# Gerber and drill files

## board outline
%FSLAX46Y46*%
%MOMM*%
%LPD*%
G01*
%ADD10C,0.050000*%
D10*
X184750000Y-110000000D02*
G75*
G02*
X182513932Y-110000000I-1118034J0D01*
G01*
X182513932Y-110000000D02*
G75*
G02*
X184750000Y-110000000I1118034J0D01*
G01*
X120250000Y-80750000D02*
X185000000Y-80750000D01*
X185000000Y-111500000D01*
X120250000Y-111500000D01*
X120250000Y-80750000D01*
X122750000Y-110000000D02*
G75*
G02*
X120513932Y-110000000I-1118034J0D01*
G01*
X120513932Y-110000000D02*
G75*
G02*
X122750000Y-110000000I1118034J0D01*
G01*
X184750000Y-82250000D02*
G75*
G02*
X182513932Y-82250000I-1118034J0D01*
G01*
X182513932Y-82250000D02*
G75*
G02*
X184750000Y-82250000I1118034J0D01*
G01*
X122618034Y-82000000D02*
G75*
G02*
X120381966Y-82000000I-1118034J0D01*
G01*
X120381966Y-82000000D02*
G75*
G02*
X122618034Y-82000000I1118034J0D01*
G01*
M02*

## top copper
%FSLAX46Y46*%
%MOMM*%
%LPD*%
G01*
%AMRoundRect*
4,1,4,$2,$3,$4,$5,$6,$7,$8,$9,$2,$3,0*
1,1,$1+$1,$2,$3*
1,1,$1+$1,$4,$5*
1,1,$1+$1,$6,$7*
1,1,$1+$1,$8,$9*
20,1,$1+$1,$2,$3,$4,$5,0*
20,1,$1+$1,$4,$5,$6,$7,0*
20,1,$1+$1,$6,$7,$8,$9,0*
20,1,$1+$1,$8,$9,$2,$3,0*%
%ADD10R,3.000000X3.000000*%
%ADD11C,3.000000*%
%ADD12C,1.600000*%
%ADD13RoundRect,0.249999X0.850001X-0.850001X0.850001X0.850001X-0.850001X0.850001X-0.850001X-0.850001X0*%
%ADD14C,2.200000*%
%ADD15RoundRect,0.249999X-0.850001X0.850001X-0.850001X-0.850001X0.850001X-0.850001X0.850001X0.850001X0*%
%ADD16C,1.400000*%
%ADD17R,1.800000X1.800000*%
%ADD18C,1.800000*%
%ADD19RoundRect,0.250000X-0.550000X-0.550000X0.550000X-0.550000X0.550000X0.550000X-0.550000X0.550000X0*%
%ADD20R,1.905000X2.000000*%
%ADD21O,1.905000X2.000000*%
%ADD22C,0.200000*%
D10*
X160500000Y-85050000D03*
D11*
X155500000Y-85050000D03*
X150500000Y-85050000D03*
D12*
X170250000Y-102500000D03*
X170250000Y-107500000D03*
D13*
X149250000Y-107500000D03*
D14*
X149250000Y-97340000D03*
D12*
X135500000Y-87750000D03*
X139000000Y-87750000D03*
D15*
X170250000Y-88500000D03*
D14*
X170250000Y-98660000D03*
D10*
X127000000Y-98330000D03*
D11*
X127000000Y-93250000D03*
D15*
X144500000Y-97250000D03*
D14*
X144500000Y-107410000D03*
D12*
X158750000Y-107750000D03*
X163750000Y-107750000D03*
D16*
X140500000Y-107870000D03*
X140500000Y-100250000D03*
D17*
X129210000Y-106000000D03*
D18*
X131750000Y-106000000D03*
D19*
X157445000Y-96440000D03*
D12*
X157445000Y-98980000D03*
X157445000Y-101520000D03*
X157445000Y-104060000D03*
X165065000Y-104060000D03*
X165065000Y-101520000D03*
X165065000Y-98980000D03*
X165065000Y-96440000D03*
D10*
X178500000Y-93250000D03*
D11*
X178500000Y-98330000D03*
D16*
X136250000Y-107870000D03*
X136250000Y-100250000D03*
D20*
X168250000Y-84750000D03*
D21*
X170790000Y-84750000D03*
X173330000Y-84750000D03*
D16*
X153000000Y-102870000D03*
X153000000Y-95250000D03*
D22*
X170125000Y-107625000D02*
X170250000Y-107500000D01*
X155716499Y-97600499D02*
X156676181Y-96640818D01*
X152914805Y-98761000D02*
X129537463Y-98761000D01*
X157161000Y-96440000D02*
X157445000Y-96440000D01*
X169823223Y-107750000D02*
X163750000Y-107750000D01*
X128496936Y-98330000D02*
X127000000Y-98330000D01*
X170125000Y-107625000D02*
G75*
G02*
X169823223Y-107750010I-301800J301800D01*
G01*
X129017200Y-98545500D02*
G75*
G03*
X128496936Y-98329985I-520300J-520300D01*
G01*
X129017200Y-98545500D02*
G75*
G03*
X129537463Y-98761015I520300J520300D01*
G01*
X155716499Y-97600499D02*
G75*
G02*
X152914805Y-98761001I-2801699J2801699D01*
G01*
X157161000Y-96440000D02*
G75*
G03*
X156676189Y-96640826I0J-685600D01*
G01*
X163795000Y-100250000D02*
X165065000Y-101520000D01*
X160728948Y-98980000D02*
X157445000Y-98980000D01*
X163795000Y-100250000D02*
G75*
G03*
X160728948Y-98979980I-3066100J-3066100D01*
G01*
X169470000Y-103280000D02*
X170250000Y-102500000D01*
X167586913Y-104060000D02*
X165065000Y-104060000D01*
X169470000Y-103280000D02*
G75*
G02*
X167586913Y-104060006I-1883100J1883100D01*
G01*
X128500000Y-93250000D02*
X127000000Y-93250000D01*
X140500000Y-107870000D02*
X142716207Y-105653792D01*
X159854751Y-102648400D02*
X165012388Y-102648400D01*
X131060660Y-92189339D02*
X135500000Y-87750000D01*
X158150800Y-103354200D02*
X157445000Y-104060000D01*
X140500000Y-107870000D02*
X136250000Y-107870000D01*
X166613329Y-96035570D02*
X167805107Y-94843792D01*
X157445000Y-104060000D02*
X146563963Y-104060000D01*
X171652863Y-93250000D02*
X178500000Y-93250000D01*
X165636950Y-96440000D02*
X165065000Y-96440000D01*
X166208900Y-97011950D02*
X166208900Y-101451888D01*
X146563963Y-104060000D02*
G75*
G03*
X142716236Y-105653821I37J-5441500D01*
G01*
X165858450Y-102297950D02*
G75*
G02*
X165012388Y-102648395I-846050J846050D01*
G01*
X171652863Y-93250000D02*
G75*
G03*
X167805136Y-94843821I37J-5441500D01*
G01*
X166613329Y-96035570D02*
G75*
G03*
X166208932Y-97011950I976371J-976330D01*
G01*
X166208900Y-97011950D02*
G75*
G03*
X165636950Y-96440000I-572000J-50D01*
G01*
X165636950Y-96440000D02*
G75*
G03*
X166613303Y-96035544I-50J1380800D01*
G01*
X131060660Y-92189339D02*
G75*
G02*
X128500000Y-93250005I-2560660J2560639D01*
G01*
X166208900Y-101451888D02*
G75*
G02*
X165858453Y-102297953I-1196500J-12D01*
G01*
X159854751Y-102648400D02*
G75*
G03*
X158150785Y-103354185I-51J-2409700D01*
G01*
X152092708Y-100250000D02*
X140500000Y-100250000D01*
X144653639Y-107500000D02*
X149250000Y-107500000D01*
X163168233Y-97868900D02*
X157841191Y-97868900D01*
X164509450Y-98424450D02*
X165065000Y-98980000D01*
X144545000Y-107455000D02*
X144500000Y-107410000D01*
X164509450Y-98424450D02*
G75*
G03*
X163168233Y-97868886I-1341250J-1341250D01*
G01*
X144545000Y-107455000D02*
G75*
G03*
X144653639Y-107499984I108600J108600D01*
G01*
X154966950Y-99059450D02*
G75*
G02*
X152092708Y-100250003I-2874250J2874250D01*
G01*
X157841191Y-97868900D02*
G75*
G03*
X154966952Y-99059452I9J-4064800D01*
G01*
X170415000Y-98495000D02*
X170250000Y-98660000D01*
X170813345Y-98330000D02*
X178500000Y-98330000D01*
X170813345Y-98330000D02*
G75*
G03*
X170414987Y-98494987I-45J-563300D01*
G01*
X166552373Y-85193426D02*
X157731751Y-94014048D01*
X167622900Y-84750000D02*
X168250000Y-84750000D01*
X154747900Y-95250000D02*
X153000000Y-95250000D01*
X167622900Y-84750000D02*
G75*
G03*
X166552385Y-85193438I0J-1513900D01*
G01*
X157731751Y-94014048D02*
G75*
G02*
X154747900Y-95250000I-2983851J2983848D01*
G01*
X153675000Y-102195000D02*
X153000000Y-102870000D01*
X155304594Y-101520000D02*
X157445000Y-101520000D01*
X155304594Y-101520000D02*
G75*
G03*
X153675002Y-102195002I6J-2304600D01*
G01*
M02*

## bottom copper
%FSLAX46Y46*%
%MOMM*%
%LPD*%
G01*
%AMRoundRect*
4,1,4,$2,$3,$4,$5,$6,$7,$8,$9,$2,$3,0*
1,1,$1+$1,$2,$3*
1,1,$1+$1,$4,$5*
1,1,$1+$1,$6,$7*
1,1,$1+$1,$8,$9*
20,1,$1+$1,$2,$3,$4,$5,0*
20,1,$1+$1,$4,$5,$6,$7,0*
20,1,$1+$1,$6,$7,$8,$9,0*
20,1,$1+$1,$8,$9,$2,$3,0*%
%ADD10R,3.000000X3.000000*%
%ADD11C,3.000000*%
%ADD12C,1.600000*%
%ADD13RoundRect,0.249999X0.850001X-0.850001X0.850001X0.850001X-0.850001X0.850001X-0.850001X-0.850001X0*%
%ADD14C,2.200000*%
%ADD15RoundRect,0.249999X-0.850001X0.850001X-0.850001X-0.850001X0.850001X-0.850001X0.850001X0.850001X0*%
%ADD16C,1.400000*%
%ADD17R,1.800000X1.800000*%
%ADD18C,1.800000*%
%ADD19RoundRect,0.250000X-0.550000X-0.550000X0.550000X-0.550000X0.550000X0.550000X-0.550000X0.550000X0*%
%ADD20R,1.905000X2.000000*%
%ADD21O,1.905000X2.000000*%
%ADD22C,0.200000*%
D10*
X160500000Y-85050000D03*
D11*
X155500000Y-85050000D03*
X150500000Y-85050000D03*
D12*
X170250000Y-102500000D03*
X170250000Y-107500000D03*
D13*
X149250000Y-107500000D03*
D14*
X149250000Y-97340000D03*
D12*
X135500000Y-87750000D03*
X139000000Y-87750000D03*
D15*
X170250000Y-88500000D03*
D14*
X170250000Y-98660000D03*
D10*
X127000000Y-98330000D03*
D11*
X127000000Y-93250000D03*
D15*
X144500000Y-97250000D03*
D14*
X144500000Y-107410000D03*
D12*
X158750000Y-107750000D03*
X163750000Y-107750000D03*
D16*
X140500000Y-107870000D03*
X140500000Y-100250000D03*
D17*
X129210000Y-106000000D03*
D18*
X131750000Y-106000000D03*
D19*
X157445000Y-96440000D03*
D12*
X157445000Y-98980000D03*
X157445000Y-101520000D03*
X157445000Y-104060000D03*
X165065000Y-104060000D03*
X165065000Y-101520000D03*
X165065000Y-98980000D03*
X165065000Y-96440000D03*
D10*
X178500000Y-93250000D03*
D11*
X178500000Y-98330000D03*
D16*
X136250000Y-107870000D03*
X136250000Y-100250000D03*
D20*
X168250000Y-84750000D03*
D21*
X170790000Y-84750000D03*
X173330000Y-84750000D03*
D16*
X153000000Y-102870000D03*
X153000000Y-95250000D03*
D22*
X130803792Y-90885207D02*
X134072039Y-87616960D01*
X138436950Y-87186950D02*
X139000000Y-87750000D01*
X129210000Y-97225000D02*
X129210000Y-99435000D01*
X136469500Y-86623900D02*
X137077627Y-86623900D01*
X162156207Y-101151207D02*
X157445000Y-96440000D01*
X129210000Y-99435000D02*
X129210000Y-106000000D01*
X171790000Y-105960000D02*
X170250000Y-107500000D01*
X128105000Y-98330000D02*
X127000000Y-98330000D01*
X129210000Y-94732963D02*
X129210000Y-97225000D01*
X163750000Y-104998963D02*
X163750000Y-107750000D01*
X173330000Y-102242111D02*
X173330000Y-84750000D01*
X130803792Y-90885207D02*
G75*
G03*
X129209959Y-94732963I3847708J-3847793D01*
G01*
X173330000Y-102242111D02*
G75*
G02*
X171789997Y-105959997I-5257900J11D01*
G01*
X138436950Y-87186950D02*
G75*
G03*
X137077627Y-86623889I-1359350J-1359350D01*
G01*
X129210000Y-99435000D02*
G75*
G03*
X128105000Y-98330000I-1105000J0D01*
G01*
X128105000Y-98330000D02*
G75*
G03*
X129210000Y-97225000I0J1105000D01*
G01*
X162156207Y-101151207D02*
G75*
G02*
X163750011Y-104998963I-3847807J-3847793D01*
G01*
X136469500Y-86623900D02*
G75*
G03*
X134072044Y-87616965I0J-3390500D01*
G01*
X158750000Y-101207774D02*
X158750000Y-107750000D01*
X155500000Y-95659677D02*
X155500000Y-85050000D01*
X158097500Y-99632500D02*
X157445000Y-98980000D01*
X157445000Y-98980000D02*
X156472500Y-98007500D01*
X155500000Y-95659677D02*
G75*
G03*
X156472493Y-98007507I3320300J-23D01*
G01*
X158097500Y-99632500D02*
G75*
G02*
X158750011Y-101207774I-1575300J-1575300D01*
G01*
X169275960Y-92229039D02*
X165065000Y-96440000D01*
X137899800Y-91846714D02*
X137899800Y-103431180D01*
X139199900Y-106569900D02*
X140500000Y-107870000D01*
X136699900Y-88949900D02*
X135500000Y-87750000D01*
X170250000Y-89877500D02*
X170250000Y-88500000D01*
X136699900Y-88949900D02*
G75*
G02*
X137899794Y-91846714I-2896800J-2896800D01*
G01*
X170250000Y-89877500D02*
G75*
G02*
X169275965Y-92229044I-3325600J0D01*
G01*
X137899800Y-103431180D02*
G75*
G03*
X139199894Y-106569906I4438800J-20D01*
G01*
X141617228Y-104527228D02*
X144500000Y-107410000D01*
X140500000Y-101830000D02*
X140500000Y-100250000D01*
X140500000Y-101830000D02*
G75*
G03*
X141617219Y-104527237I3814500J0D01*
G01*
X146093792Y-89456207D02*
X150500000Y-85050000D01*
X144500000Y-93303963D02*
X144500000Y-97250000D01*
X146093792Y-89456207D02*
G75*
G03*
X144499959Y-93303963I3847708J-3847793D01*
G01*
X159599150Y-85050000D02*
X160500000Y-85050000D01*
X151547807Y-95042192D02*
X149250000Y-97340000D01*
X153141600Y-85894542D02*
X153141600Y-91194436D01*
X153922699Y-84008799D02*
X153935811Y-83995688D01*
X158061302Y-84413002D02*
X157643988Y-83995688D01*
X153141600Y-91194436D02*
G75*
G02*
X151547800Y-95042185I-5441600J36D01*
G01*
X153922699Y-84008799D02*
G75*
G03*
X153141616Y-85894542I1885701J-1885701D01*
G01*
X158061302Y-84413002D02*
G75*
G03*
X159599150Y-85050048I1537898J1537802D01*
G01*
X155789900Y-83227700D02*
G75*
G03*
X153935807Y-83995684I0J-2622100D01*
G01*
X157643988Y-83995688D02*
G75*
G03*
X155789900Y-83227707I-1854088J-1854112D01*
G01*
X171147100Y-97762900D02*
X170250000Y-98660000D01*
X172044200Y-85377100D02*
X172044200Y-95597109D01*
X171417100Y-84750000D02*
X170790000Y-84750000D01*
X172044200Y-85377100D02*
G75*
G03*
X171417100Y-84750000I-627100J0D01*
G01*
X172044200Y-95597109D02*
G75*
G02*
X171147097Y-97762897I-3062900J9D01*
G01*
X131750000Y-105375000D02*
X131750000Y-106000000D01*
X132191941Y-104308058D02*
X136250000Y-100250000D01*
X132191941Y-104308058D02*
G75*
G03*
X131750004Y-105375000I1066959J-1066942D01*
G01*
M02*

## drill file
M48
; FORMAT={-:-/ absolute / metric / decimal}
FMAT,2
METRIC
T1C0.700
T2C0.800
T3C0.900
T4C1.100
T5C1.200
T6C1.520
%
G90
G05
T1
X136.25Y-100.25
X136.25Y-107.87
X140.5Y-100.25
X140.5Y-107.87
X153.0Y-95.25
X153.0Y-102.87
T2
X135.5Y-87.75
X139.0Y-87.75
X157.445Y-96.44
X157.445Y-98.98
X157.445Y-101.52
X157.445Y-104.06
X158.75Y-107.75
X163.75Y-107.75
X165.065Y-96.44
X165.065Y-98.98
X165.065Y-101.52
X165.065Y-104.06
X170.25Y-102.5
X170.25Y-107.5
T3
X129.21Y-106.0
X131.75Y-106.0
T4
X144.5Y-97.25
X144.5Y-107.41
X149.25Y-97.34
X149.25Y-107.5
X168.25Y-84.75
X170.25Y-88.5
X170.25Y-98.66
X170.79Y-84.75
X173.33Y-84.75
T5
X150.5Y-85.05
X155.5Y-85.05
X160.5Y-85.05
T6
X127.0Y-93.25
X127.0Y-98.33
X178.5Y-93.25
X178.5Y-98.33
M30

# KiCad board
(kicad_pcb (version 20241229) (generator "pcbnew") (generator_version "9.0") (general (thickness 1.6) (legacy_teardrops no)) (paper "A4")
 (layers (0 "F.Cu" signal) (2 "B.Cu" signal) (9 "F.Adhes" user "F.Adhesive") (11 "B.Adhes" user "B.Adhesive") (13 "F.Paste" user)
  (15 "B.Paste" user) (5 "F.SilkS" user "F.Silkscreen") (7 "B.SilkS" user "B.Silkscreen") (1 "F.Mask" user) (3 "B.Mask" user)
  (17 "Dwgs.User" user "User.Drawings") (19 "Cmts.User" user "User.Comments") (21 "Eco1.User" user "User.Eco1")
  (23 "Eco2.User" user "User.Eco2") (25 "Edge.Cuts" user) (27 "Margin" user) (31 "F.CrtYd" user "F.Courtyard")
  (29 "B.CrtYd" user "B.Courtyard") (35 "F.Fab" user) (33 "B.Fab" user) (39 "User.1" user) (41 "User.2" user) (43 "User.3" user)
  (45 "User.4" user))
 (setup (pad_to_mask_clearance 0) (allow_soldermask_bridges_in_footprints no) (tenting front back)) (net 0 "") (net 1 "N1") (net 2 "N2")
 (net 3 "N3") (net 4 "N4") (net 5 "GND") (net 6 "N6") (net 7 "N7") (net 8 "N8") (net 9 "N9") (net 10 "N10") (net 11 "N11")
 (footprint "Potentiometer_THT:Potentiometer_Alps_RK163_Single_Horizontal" (layer "F.Cu") (at 160.5 85.05 -90)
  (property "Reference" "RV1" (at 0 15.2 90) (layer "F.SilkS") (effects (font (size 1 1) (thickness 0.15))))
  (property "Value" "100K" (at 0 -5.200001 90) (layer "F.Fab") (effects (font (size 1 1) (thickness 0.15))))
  (pad "1" thru_hole rect (at 0 0 90) (size 3 3) (drill 1.2) (layers "*.Cu" "*.Mask") (remove_unused_layers no) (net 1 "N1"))
  (pad "2" thru_hole circle (at 0 5 90) (size 3 3) (drill 1.2) (layers "*.Cu" "*.Mask") (remove_unused_layers no) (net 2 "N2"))
  (pad "3" thru_hole circle (at 0 10 90) (size 3 3) (drill 1.2) (layers "*.Cu" "*.Mask") (remove_unused_layers no) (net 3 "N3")))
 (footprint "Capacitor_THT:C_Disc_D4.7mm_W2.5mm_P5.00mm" (layer "F.Cu") (at 170.25 102.5 -90)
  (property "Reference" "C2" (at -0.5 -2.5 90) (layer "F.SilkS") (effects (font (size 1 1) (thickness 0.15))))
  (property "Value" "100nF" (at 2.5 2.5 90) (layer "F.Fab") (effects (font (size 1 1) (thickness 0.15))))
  (pad "1" thru_hole circle (at 0 0 270) (size 1.6 1.6) (drill 0.8) (layers "*.Cu" "*.Mask") (remove_unused_layers no) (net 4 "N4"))
  (pad "2" thru_hole circle (at 5 0 270) (size 1.6 1.6) (drill 0.8) (layers "*.Cu" "*.Mask") (remove_unused_layers no) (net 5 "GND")))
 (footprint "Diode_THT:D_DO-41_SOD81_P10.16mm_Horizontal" (layer "F.Cu") (at 149.25 107.5 90)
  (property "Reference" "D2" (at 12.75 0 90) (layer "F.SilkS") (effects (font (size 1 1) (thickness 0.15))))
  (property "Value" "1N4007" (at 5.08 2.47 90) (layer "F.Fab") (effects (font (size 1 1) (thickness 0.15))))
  (pad "1" thru_hole roundrect (at 0 0 90) (size 2.2 2.2) (drill 1.1) (layers "*.Cu" "*.Mask") (remove_unused_layers no)
   (roundrect_rratio 0.113636) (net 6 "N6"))
  (pad "2" thru_hole circle (at 10.16 0 90) (size 2.2 2.2) (drill 1.1) (layers "*.Cu" "*.Mask") (remove_unused_layers no) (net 1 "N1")))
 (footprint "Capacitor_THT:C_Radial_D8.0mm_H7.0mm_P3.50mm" (layer "F.Cu") (at 135.5 87.75)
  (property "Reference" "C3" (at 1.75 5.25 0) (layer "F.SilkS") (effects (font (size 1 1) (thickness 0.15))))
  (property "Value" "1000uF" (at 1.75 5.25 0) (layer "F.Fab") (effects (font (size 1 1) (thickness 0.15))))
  (pad "1" thru_hole circle (at 0 0) (size 1.6 1.6) (drill 0.8) (layers "*.Cu" "*.Mask") (remove_unused_layers no) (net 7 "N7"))
  (pad "2" thru_hole circle (at 3.5 0) (size 1.6 1.6) (drill 0.8) (layers "*.Cu" "*.Mask") (remove_unused_layers no) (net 5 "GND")))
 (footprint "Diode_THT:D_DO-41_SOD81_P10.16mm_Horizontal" (layer "F.Cu") (at 170.25 88.5 -90)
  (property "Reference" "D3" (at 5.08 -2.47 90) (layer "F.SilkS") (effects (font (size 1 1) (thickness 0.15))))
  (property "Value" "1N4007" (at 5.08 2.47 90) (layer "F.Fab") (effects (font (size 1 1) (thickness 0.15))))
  (pad "1" thru_hole roundrect (at 0 0 270) (size 2.2 2.2) (drill 1.1) (layers "*.Cu" "*.Mask") (remove_unused_layers no)
   (roundrect_rratio 0.113636) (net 7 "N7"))
  (pad "2" thru_hole circle (at 10.16 0 270) (size 2.2 2.2) (drill 1.1) (layers "*.Cu" "*.Mask") (remove_unused_layers no) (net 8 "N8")))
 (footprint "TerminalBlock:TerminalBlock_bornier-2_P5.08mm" (layer "F.Cu") (at 127 98.33 90)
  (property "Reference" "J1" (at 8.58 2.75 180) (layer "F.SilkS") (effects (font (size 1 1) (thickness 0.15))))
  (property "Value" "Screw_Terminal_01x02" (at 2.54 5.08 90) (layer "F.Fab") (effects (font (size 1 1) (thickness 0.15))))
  (pad "1" thru_hole rect (at 0 0 90) (size 3 3) (drill 1.52) (layers "*.Cu" "*.Mask") (remove_unused_layers no) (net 5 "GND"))
  (pad "2" thru_hole circle (at 5.08 0 90) (size 3 3) (drill 1.52) (layers "*.Cu" "*.Mask") (remove_unused_layers no) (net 7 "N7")))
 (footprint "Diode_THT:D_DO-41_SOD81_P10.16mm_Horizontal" (layer "F.Cu") (at 144.5 97.25 -90)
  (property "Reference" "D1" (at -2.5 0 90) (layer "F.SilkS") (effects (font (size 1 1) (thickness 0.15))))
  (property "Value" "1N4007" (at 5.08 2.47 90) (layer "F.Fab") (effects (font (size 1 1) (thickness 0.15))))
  (pad "1" thru_hole roundrect (at 0 0 270) (size 2.2 2.2) (drill 1.1) (layers "*.Cu" "*.Mask") (remove_unused_layers no)
   (roundrect_rratio 0.113636) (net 3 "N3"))
  (pad "2" thru_hole circle (at 10.16 0 270) (size 2.2 2.2) (drill 1.1) (layers "*.Cu" "*.Mask") (remove_unused_layers no) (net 6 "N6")))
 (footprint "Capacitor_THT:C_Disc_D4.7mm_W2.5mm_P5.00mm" (layer "F.Cu") (at 158.75 107.75)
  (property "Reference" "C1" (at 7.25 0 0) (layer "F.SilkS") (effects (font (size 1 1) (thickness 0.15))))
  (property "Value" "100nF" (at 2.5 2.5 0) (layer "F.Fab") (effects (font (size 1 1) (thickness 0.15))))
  (pad "1" thru_hole circle (at 0 0) (size 1.6 1.6) (drill 0.8) (layers "*.Cu" "*.Mask") (remove_unused_layers no) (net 2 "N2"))
  (pad "2" thru_hole circle (at 5 0) (size 1.6 1.6) (drill 0.8) (layers "*.Cu" "*.Mask") (remove_unused_layers no) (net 5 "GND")))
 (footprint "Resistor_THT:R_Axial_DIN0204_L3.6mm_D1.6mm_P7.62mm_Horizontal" (layer "F.Cu") (at 140.5 107.87 90)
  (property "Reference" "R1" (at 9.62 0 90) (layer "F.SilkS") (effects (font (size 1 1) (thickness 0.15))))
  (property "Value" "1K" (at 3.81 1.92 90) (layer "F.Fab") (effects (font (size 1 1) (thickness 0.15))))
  (pad "1" thru_hole circle (at 0 0 90) (size 1.4 1.4) (drill 0.7) (layers "*.Cu" "*.Mask") (remove_unused_layers no) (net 7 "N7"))
  (pad "2" thru_hole circle (at 7.62 0 90) (size 1.4 1.4) (drill 0.7) (layers "*.Cu" "*.Mask") (remove_unused_layers no) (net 6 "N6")))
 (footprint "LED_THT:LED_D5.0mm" (layer "F.Cu") (at 129.21 106)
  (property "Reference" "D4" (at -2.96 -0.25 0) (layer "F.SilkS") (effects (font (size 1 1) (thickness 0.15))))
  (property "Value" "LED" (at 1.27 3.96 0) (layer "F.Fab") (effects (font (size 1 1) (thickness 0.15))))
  (pad "1" thru_hole rect (at 0 0) (size 1.8 1.8) (drill 0.9) (layers "*.Cu" "*.Mask") (remove_unused_layers no) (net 5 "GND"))
  (pad "2" thru_hole circle (at 2.54 0) (size 1.8 1.8) (drill 0.9) (layers "*.Cu" "*.Mask") (remove_unused_layers no) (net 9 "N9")))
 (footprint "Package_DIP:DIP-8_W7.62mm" (layer "F.Cu") (at 157.445 96.44)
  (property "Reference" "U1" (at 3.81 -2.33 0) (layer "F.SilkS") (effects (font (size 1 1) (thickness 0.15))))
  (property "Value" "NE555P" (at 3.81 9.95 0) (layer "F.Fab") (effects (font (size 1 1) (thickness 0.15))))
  (pad "1" thru_hole roundrect (at 0 0) (size 1.6 1.6) (drill 0.8) (layers "*.Cu" "*.Mask") (remove_unused_layers no)
   (roundrect_rratio 0.15625) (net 5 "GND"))
  (pad "2" thru_hole circle (at 0 2.54) (size 1.6 1.6) (drill 0.8) (layers "*.Cu" "*.Mask") (remove_unused_layers no) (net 2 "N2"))
  (pad "3" thru_hole circle (at 0 5.08) (size 1.6 1.6) (drill 0.8) (layers "*.Cu" "*.Mask") (remove_unused_layers no) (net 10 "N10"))
  (pad "4" thru_hole circle (at 0 7.62) (size 1.6 1.6) (drill 0.8) (layers "*.Cu" "*.Mask") (remove_unused_layers no) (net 7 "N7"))
  (pad "5" thru_hole circle (at 7.62 7.62) (size 1.6 1.6) (drill 0.8) (layers "*.Cu" "*.Mask") (remove_unused_layers no) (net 4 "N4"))
  (pad "6" thru_hole circle (at 7.62 5.08) (size 1.6 1.6) (drill 0.8) (layers "*.Cu" "*.Mask") (remove_unused_layers no) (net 2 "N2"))
  (pad "7" thru_hole circle (at 7.62 2.54) (size 1.6 1.6) (drill 0.8) (layers "*.Cu" "*.Mask") (remove_unused_layers no) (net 6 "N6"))
  (pad "8" thru_hole circle (at 7.62 0) (size 1.6 1.6) (drill 0.8) (layers "*.Cu" "*.Mask") (remove_unused_layers no) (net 7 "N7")))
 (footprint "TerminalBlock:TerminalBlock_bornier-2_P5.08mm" (layer "F.Cu") (at 178.5 93.25 -90)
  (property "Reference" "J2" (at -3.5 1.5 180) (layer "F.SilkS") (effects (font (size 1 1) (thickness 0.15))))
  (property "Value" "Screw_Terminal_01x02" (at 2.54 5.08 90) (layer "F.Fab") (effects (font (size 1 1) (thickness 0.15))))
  (pad "1" thru_hole rect (at 0 0 270) (size 3 3) (drill 1.52) (layers "*.Cu" "*.Mask") (remove_unused_layers no) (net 7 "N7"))
  (pad "2" thru_hole circle (at 5.08 0 270) (size 3 3) (drill 1.52) (layers "*.Cu" "*.Mask") (remove_unused_layers no) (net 8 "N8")))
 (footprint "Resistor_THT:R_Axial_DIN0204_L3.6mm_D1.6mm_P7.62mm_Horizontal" (layer "F.Cu") (at 136.25 107.87 90)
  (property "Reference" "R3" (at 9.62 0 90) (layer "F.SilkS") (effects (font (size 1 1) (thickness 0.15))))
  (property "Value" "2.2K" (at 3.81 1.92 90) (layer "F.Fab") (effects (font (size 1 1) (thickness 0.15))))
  (pad "1" thru_hole circle (at 0 0 90) (size 1.4 1.4) (drill 0.7) (layers "*.Cu" "*.Mask") (remove_unused_layers no) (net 7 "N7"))
  (pad "2" thru_hole circle (at 7.62 0 90) (size 1.4 1.4) (drill 0.7) (layers "*.Cu" "*.Mask") (remove_unused_layers no) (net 9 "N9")))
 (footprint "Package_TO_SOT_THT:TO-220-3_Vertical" (layer "F.Cu") (at 168.25 84.75)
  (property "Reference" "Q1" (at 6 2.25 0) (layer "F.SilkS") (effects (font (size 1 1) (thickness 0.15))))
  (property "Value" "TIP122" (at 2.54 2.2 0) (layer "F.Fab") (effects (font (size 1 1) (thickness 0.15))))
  (pad "1" thru_hole rect (at 0 0) (size 1.905 2) (drill 1.1) (layers "*.Cu" "*.Mask") (remove_unused_layers no) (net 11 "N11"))
  (pad "2" thru_hole oval (at 2.54 0) (size 1.905 2) (drill 1.1) (layers "*.Cu" "*.Mask") (remove_unused_layers no) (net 8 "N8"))
  (pad "3" thru_hole oval (at 5.08 0) (size 1.905 2) (drill 1.1) (layers "*.Cu" "*.Mask") (remove_unused_layers no) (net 5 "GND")))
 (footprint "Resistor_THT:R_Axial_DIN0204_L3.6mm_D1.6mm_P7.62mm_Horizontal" (layer "F.Cu") (at 153 102.87 90)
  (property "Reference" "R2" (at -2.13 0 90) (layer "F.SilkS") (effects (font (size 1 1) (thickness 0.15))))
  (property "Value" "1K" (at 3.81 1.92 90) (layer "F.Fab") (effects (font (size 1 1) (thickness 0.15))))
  (pad "1" thru_hole circle (at 0 0 90) (size 1.4 1.4) (drill 0.7) (layers "*.Cu" "*.Mask") (remove_unused_layers no) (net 10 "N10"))
  (pad "2" thru_hole circle (at 7.62 0 90) (size 1.4 1.4) (drill 0.7) (layers "*.Cu" "*.Mask") (remove_unused_layers no) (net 11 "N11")))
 (gr_circle (center 183.631966 110) (end 182.631966 109.5) (stroke (width 0.05) (type default)) (fill no) (layer "Edge.Cuts"))
 (gr_rect (start 120.25 80.75) (end 185 111.5) (stroke (width 0.05) (type default)) (fill no) (layer "Edge.Cuts"))
 (gr_circle (center 121.631966 110) (end 120.631966 109.5) (stroke (width 0.05) (type default)) (fill no) (layer "Edge.Cuts"))
 (gr_circle (center 183.631966 82.25) (end 182.631966 81.75) (stroke (width 0.05) (type default)) (fill no) (layer "Edge.Cuts"))
 (gr_circle (center 121.5 82) (end 120.5 81.5) (stroke (width 0.05) (type default)) (fill no) (layer "Edge.Cuts"))
 (segment (start 170.125 107.625) (end 170.25 107.5) (width 0.2) (layer "F.Cu") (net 5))
 (segment (start 155.716499 97.600499) (end 156.676181 96.640818) (width 0.2) (layer "F.Cu") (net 5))
 (segment (start 152.914805 98.761) (end 129.537463 98.761) (width 0.2) (layer "F.Cu") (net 5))
 (segment (start 157.161 96.44) (end 157.445 96.44) (width 0.2) (layer "F.Cu") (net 5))
 (segment (start 169.823223 107.75) (end 163.75 107.75) (width 0.2) (layer "F.Cu") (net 5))
 (segment (start 128.496936 98.33) (end 127 98.33) (width 0.2) (layer "F.Cu") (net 5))
 (arc (start 170.125 107.625) (mid 169.986543 107.717513) (end 169.823223 107.75) (width 0.2) (layer "F.Cu") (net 5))
 (arc (start 129.0172 98.5455) (mid 128.778501 98.386006) (end 128.496936 98.33) (width 0.2) (layer "F.Cu") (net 5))
 (arc (start 129.0172 98.5455) (mid 129.255898 98.704993) (end 129.537463 98.761) (width 0.2) (layer "F.Cu") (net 5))
 (arc (start 155.716499 97.600499) (mid 154.431071 98.459395) (end 152.914805 98.761) (width 0.2) (layer "F.Cu") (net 5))
 (arc (start 157.161 96.44) (mid 156.898618 96.49219) (end 156.676181 96.640818) (width 0.2) (layer "F.Cu") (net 5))
 (segment (start 130.803792 90.885207) (end 134.072039 87.61696) (width 0.2) (layer "B.Cu") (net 5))
 (segment (start 138.43695 87.18695) (end 139 87.75) (width 0.2) (layer "B.Cu") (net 5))
 (segment (start 129.21 97.225) (end 129.21 99.435) (width 0.2) (layer "B.Cu") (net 5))
 (segment (start 136.4695 86.6239) (end 137.077627 86.6239) (width 0.2) (layer "B.Cu") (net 5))
 (segment (start 162.156207 101.151207) (end 157.445 96.44) (width 0.2) (layer "B.Cu") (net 5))
 (segment (start 129.21 99.435) (end 129.21 106) (width 0.2) (layer "B.Cu") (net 5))
 (segment (start 171.79 105.96) (end 170.25 107.5) (width 0.2) (layer "B.Cu") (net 5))
 (segment (start 128.105 98.33) (end 127 98.33) (width 0.2) (layer "B.Cu") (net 5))
 (segment (start 129.21 94.732963) (end 129.21 97.225) (width 0.2) (layer "B.Cu") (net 5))
 (segment (start 163.75 104.998963) (end 163.75 107.75) (width 0.2) (layer "B.Cu") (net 5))
 (segment (start 173.33 102.242111) (end 173.33 84.75) (width 0.2) (layer "B.Cu") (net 5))
 (arc (start 130.803792 90.885207) (mid 129.624213 92.650572) (end 129.21 94.732963) (width 0.2) (layer "B.Cu") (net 5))
 (arc (start 173.33 102.242111) (mid 172.929767 104.254218) (end 171.79 105.96) (width 0.2) (layer "B.Cu") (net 5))
 (arc (start 138.43695 87.18695) (mid 137.813287 86.770231) (end 137.077627 86.6239) (width 0.2) (layer "B.Cu") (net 5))
 (arc (start 129.21 99.435) (mid 128.886352 98.653647) (end 128.105 98.33) (width 0.2) (layer "B.Cu") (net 5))
 (arc (start 128.105 98.33) (mid 128.886352 98.006352) (end 129.21 97.225) (width 0.2) (layer "B.Cu") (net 5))
 (arc (start 162.156207 101.151207) (mid 163.335786 102.916572) (end 163.75 104.998963) (width 0.2) (layer "B.Cu") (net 5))
 (arc (start 136.4695 86.6239) (mid 135.172003 86.881987) (end 134.072039 87.61696) (width 0.2) (layer "B.Cu") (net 5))
 (segment (start 163.795 100.25) (end 165.065 101.52) (width 0.2) (layer "F.Cu") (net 2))
 (segment (start 160.728948 98.98) (end 157.445 98.98) (width 0.2) (layer "F.Cu") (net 2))
 (arc (start 163.795 100.25) (mid 162.388283 99.310062) (end 160.728948 98.98) (width 0.2) (layer "F.Cu") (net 2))
 (segment (start 158.75 101.207774) (end 158.75 107.75) (width 0.2) (layer "B.Cu") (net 2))
 (segment (start 155.5 95.659677) (end 155.5 85.05) (width 0.2) (layer "B.Cu") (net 2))
 (segment (start 158.0975 99.6325) (end 157.445 98.98) (width 0.2) (layer "B.Cu") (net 2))
 (segment (start 157.445 98.98) (end 156.4725 98.0075) (width 0.2) (layer "B.Cu") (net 2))
 (arc (start 155.5 95.659677) (mid 155.752744 96.930309) (end 156.4725 98.0075) (width 0.2) (layer "B.Cu") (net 2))
 (arc (start 158.0975 99.6325) (mid 158.58042 100.355241) (end 158.75 101.207774) (width 0.2) (layer "B.Cu") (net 2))
 (segment (start 169.47 103.28) (end 170.25 102.5) (width 0.2) (layer "F.Cu") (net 4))
 (segment (start 167.586913 104.06) (end 165.065 104.06) (width 0.2) (layer "F.Cu") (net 4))
 (arc (start 169.47 103.28) (mid 168.606032 103.857284) (end 167.586913 104.06) (width 0.2) (layer "F.Cu") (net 4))
 (segment (start 128.5 93.25) (end 127 93.25) (width 0.2) (layer "F.Cu") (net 7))
 (segment (start 140.5 107.87) (end 142.716207 105.653792) (width 0.2) (layer "F.Cu") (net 7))
 (segment (start 159.854751 102.6484) (end 165.012388 102.6484) (width 0.2) (layer "F.Cu") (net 7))
 (segment (start 131.06066 92.189339) (end 135.5 87.75) (width 0.2) (layer "F.Cu") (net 7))
 (segment (start 158.1508 103.3542) (end 157.445 104.06) (width 0.2) (layer "F.Cu") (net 7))
 (segment (start 140.5 107.87) (end 136.25 107.87) (width 0.2) (layer "F.Cu") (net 7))
 (segment (start 166.613329 96.03557) (end 167.805107 94.843792) (width 0.2) (layer "F.Cu") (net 7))
 (segment (start 157.445 104.06) (end 146.563963 104.06) (width 0.2) (layer "F.Cu") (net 7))
 (segment (start 171.652863 93.25) (end 178.5 93.25) (width 0.2) (layer "F.Cu") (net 7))
 (segment (start 165.63695 96.44) (end 165.065 96.44) (width 0.2) (layer "F.Cu") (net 7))
 (segment (start 166.2089 97.01195) (end 166.2089 101.451888) (width 0.2) (layer "F.Cu") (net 7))
 (arc (start 146.563963 104.06) (mid 144.481572 104.474213) (end 142.716207 105.653792) (width 0.2) (layer "F.Cu") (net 7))
 (arc (start 165.85845 102.29795) (mid 165.470273 102.557321) (end 165.012388 102.6484) (width 0.2) (layer "F.Cu") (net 7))
 (arc (start 171.652863 93.25) (mid 169.570472 93.664213) (end 167.805107 94.843792) (width 0.2) (layer "F.Cu") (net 7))
 (arc (start 166.613329 96.03557) (mid 166.314007 96.483537) (end 166.2089 97.01195) (width 0.2) (layer "F.Cu") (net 7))
 (arc (start 166.2089 97.01195) (mid 166.041379 96.60752) (end 165.63695 96.44) (width 0.2) (layer "F.Cu") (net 7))
 (arc (start 165.63695 96.44) (mid 166.165362 96.334892) (end 166.613329 96.03557) (width 0.2) (layer "F.Cu") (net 7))
 (arc (start 131.06066 92.189339) (mid 129.885819 92.974343) (end 128.5 93.25) (width 0.2) (layer "F.Cu") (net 7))
 (arc (start 166.2089 101.451888) (mid 166.117821 101.909773) (end 165.85845 102.29795) (width 0.2) (layer "F.Cu") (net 7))
 (arc (start 159.854751 102.6484) (mid 158.932579 102.831831) (end 158.1508 103.3542) (width 0.2) (layer "F.Cu") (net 7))
 (segment (start 169.27596 92.229039) (end 165.065 96.44) (width 0.2) (layer "B.Cu") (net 7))
 (segment (start 137.8998 91.846714) (end 137.8998 103.43118) (width 0.2) (layer "B.Cu") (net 7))
 (segment (start 139.1999 106.5699) (end 140.5 107.87) (width 0.2) (layer "B.Cu") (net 7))
 (segment (start 136.6999 88.9499) (end 135.5 87.75) (width 0.2) (layer "B.Cu") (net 7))
 (segment (start 170.25 89.8775) (end 170.25 88.5) (width 0.2) (layer "B.Cu") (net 7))
 (arc (start 136.6999 88.9499) (mid 137.587956 90.278969) (end 137.8998 91.846714) (width 0.2) (layer "B.Cu") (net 7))
 (arc (start 170.25 89.8775) (mid 169.996855 91.150143) (end 169.27596 92.229039) (width 0.2) (layer "B.Cu") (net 7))
 (arc (start 137.8998 103.43118) (mid 138.237684 105.129843) (end 139.1999 106.5699) (width 0.2) (layer "B.Cu") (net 7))
 (segment (start 152.092708 100.25) (end 140.5 100.25) (width 0.2) (layer "F.Cu") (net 6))
 (segment (start 144.653639 107.5) (end 149.25 107.5) (width 0.2) (layer "F.Cu") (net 6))
 (segment (start 163.168233 97.8689) (end 157.841191 97.8689) (width 0.2) (layer "F.Cu") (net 6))
 (segment (start 164.50945 98.42445) (end 165.065 98.98) (width 0.2) (layer "F.Cu") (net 6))
 (segment (start 144.545 107.455) (end 144.5 107.41) (width 0.2) (layer "F.Cu") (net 6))
 (arc (start 164.50945 98.42445) (mid 163.894094 98.013282) (end 163.168233 97.8689) (width 0.2) (layer "F.Cu") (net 6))
 (arc (start 144.545 107.455) (mid 144.594844 107.488304) (end 144.653639 107.5) (width 0.2) (layer "F.Cu") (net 6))
 (arc (start 154.96695 99.05945) (mid 153.648236 99.940586) (end 152.092708 100.25) (width 0.2) (layer "F.Cu") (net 6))
 (arc (start 157.841191 97.8689) (mid 156.285663 98.178313) (end 154.96695 99.05945) (width 0.2) (layer "F.Cu") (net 6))
 (segment (start 141.617228 104.527228) (end 144.5 107.41) (width 0.2) (layer "B.Cu") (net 6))
 (segment (start 140.5 101.83) (end 140.5 100.25) (width 0.2) (layer "B.Cu") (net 6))
 (arc (start 140.5 101.83) (mid 140.790358 103.289729) (end 141.617228 104.527228) (width 0.2) (layer "B.Cu") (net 6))
 (segment (start 146.093792 89.456207) (end 150.5 85.05) (width 0.2) (layer "B.Cu") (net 3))
 (segment (start 144.5 93.303963) (end 144.5 97.25) (width 0.2) (layer "B.Cu") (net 3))
 (arc (start 146.093792 89.456207) (mid 144.914213 91.221572) (end 144.5 93.303963) (width 0.2) (layer "B.Cu") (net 3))
 (segment (start 159.59915 85.05) (end 160.5 85.05) (width 0.2) (layer "B.Cu") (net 1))
 (segment (start 151.547807 95.042192) (end 149.25 97.34) (width 0.2) (layer "B.Cu") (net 1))
 (segment (start 153.1416 85.894542) (end 153.1416 91.194436) (width 0.2) (layer "B.Cu") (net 1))
 (segment (start 153.922699 84.008799) (end 153.935811 83.995688) (width 0.2) (layer "B.Cu") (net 1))
 (segment (start 158.061302 84.413002) (end 157.643988 83.995688) (width 0.2) (layer "B.Cu") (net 1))
 (arc (start 153.1416 91.194436) (mid 152.727386 93.276826) (end 151.547807 95.042192) (width 0.2) (layer "B.Cu") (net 1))
 (arc (start 153.922699 84.008799) (mid 153.344601 84.873985) (end 153.1416 85.894542) (width 0.2) (layer "B.Cu") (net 1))
 (arc (start 158.061302 84.413002) (mid 158.766872 84.884449) (end 159.59915 85.05) (width 0.2) (layer "B.Cu") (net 1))
 (arc (start 155.7899 83.2277) (mid 154.786474 83.427293) (end 153.935811 83.995688) (width 0.2) (layer "B.Cu") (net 1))
 (arc (start 157.643988 83.995688) (mid 156.793325 83.427293) (end 155.7899 83.2277) (width 0.2) (layer "B.Cu") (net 1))
 (segment (start 170.415 98.495) (end 170.25 98.66) (width 0.2) (layer "F.Cu") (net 8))
 (segment (start 170.813345 98.33) (end 178.5 98.33) (width 0.2) (layer "F.Cu") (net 8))
 (arc (start 170.813345 98.33) (mid 170.597762 98.372882) (end 170.415 98.495) (width 0.2) (layer "F.Cu") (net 8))
 (segment (start 171.1471 97.7629) (end 170.25 98.66) (width 0.2) (layer "B.Cu") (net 8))
 (segment (start 172.0442 85.3771) (end 172.0442 95.597109) (width 0.2) (layer "B.Cu") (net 8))
 (segment (start 171.4171 84.75) (end 170.79 84.75) (width 0.2) (layer "B.Cu") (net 8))
 (arc (start 172.0442 85.3771) (mid 171.860526 84.933673) (end 171.4171 84.75) (width 0.2) (layer "B.Cu") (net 8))
 (arc (start 172.0442 95.597109) (mid 171.811051 96.769226) (end 171.1471 97.7629) (width 0.2) (layer "B.Cu") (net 8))
 (segment (start 131.75 105.375) (end 131.75 106) (width 0.2) (layer "B.Cu") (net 9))
 (segment (start 132.191941 104.308058) (end 136.25 100.25) (width 0.2) (layer "B.Cu") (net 9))
 (arc (start 132.191941 104.308058) (mid 131.864856 104.797575) (end 131.75 105.375) (width 0.2) (layer "B.Cu") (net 9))
 (segment (start 166.552373 85.193426) (end 157.731751 94.014048) (width 0.2) (layer "F.Cu") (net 11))
 (segment (start 167.6229 84.75) (end 168.25 84.75) (width 0.2) (layer "F.Cu") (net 11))
 (segment (start 154.7479 95.25) (end 153 95.25) (width 0.2) (layer "F.Cu") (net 11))
 (arc (start 167.6229 84.75) (mid 167.043535 84.865242) (end 166.552373 85.193426) (width 0.2) (layer "F.Cu") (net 11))
 (arc (start 157.731751 94.014048) (mid 156.362748 94.928786) (end 154.7479 95.25) (width 0.2) (layer "F.Cu") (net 11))
 (segment (start 153.675 102.195) (end 153 102.87) (width 0.2) (layer "F.Cu") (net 10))
 (segment (start 155.304594 101.52) (end 157.445 101.52) (width 0.2) (layer "F.Cu") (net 10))
 (arc (start 155.304594 101.52) (mid 154.422664 101.695426) (end 153.675 102.195) (width 0.2) (layer "F.Cu") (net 10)))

